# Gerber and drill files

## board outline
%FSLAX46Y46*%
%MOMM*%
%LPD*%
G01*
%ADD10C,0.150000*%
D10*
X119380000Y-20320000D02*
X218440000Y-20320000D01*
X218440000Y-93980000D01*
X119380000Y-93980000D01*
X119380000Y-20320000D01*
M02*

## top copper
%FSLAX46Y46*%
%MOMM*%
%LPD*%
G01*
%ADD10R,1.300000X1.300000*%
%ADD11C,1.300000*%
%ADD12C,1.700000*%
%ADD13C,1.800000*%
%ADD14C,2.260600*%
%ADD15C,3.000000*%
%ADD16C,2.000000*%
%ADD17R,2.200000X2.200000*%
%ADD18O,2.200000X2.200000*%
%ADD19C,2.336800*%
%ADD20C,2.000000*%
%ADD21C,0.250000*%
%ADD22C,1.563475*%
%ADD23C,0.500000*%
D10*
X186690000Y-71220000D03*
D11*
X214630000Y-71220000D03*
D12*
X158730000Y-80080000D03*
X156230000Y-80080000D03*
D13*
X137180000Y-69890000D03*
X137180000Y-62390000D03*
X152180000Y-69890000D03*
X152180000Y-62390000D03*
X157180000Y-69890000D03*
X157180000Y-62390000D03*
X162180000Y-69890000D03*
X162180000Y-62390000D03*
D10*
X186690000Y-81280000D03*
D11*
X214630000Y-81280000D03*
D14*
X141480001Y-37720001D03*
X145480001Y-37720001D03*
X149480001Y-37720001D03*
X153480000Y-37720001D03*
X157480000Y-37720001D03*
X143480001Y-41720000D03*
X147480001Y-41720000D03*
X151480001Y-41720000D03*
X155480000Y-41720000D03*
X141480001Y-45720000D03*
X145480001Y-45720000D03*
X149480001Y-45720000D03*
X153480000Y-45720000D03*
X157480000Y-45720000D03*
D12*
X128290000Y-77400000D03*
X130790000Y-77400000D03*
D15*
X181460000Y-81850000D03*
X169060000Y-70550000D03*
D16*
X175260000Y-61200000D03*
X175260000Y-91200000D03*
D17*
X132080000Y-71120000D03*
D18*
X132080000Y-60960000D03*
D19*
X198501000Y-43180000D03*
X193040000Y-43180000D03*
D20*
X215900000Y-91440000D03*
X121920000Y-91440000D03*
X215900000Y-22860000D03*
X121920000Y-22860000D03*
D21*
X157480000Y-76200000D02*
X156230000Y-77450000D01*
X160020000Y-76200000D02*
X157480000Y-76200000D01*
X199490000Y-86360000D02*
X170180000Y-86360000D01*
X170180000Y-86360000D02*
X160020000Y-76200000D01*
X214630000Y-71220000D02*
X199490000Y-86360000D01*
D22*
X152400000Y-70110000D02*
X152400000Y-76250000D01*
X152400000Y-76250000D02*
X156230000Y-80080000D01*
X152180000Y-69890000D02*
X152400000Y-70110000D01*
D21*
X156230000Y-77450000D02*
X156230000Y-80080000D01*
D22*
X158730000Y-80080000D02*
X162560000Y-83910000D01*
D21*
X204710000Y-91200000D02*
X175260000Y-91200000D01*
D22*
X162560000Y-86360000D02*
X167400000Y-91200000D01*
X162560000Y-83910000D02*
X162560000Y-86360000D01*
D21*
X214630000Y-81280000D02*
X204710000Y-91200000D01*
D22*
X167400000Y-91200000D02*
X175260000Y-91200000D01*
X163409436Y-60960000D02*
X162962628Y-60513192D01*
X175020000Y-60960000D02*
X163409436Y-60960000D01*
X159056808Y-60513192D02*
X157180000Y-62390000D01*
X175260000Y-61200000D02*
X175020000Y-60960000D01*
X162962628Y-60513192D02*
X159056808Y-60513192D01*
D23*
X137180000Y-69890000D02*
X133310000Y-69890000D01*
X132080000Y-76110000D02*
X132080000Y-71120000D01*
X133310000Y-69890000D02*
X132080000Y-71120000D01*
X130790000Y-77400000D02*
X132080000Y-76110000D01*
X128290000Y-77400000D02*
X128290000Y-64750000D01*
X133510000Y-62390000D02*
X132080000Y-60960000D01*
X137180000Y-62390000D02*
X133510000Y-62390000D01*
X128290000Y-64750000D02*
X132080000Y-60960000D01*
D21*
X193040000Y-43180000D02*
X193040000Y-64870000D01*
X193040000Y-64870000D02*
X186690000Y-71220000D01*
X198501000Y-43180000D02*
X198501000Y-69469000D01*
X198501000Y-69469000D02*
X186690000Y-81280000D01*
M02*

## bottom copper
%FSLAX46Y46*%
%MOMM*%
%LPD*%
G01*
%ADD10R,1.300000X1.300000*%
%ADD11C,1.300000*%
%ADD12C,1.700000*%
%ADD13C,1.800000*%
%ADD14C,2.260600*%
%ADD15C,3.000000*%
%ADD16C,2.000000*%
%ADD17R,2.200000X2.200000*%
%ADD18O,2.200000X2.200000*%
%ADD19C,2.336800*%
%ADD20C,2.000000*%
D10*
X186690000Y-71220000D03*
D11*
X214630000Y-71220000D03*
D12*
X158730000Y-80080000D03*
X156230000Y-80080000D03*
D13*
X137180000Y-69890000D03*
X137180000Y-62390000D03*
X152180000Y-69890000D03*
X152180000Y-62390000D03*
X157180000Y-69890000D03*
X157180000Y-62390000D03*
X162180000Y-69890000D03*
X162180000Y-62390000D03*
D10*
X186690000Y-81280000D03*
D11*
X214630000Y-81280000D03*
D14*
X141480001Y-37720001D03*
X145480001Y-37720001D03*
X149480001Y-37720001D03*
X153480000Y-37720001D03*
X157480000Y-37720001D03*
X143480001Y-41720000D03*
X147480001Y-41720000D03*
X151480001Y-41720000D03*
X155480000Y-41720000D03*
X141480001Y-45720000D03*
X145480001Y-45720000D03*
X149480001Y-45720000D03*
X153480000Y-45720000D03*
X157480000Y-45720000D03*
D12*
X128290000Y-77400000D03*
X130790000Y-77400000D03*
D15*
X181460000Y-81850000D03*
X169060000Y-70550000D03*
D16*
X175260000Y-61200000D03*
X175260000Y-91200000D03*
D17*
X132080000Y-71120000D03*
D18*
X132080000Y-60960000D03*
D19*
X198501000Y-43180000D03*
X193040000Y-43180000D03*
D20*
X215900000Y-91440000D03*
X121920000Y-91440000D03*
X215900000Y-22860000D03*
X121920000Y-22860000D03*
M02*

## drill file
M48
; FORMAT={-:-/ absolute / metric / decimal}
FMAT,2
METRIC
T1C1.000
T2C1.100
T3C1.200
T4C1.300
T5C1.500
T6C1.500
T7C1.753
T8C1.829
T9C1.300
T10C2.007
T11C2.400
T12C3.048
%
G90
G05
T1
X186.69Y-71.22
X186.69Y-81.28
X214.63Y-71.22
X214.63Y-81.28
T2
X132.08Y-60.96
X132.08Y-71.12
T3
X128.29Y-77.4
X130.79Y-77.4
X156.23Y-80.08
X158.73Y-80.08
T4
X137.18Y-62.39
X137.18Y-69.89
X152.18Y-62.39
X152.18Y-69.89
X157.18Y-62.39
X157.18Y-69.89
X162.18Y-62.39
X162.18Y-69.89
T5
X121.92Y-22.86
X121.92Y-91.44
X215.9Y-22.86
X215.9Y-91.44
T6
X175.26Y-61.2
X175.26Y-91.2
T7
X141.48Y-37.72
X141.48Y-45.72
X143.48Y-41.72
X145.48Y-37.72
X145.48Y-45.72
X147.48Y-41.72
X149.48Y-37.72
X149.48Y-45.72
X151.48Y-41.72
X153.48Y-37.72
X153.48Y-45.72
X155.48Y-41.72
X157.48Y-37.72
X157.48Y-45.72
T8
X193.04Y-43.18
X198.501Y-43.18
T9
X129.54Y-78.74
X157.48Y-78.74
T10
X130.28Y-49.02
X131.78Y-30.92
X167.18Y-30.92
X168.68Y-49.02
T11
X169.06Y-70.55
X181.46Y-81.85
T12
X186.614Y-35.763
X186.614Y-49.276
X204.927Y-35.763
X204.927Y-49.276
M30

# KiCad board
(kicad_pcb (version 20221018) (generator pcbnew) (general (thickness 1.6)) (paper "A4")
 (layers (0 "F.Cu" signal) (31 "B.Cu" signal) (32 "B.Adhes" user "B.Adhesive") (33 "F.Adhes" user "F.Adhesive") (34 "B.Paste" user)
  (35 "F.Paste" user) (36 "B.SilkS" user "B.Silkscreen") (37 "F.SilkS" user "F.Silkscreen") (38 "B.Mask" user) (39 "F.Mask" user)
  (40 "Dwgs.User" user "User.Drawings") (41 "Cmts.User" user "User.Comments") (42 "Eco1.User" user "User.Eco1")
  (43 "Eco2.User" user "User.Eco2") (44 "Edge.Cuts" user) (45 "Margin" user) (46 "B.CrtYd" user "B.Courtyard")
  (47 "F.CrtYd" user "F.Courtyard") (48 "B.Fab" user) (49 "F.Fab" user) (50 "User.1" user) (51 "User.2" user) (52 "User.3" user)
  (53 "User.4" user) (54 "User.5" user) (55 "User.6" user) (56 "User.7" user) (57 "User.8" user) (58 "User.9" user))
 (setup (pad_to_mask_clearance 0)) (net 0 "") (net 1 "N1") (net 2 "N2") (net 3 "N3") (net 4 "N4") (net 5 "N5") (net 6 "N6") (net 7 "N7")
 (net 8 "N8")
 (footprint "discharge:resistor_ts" (layer "F.Cu") (at 190.627 67.4735)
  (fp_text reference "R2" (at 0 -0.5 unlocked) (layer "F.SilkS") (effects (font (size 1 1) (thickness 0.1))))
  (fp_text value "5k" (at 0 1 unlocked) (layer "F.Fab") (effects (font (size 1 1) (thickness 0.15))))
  (pad "1" thru_hole rect (at -3.937 3.7465) (size 1.3 1.3) (drill 1) (layers "*.Cu" "*.Mask") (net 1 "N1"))
  (pad "2" thru_hole circle (at 24.003 3.7465) (size 1.3 1.3) (drill 1) (layers "*.Cu" "*.Mask") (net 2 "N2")))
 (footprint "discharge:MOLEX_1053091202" (layer "F.Cu") (at 158.73 80.08 180)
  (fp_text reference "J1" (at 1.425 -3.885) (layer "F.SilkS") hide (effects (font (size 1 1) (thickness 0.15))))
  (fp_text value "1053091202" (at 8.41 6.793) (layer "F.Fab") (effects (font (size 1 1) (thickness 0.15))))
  (pad "" np_thru_hole circle (at 1.25 1.34 180) (size 1.3 1.3) (drill 1.3) (layers "*.Cu" "*.Mask"))
  (pad "1" thru_hole circle (at 0 0 180) (size 1.7 1.7) (drill 1.2) (layers "*.Cu") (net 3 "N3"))
  (pad "2" thru_hole circle (at 2.5 0 180) (size 1.7 1.7) (drill 1.2) (layers "*.Cu") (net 2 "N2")))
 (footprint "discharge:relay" (layer "F.Cu") (at 134.68 72.39 90)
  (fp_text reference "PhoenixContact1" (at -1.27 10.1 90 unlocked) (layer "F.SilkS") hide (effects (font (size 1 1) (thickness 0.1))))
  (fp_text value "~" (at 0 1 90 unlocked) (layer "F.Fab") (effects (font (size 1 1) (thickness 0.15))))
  (pad "1" thru_hole circle (at 2.5 2.5 90) (size 1.8 1.8) (drill 1.3) (layers "*.Cu" "*.Mask") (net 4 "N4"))
  (pad "2" thru_hole circle (at 10 2.5 90) (size 1.8 1.8) (drill 1.3) (layers "*.Cu" "*.Mask") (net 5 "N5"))
  (pad "3" thru_hole circle (at 2.5 17.5 90) (size 1.8 1.8) (drill 1.3) (layers "*.Cu" "*.Mask") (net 2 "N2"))
  (pad "3" thru_hole circle (at 10 17.5 90) (size 1.8 1.8) (drill 1.3) (layers "*.Cu" "*.Mask") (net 2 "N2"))
  (pad "4" thru_hole circle (at 2.5 22.5 90) (size 1.8 1.8) (drill 1.3) (layers "*.Cu" "*.Mask") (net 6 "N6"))
  (pad "4" thru_hole circle (at 10 22.5 90) (size 1.8 1.8) (drill 1.3) (layers "*.Cu" "*.Mask") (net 6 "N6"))
  (pad "5" thru_hole circle (at 2.5 27.5 90) (size 1.8 1.8) (drill 1.3) (layers "*.Cu" "*.Mask") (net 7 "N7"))
  (pad "5" thru_hole circle (at 10 27.5 90) (size 1.8 1.8) (drill 1.3) (layers "*.Cu" "*.Mask") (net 7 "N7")))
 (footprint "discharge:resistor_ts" (layer "F.Cu") (at 190.627 77.5335)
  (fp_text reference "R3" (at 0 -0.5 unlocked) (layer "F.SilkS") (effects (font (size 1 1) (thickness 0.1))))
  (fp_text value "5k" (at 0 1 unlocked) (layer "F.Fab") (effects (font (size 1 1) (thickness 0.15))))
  (pad "1" thru_hole rect (at -3.937 3.7465) (size 1.3 1.3) (drill 1) (layers "*.Cu" "*.Mask") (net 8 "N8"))
  (pad "2" thru_hole circle (at 24.003 3.7465) (size 1.3 1.3) (drill 1) (layers "*.Cu" "*.Mask") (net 3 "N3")))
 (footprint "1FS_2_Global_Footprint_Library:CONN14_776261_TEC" (layer "F.Cu") (at 157.48 45.72)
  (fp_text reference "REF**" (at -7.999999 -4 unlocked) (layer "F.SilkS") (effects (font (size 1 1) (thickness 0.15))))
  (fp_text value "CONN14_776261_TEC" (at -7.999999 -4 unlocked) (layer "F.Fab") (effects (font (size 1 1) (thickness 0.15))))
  (pad "" np_thru_hole circle (at -27.199999 3.300001) (size 2.0066 2.0066) (drill 2.0066) (layers "*.Cu" "*.Mask"))
  (pad "" np_thru_hole circle (at -25.700003 -14.799999) (size 2.0066 2.0066) (drill 2.0066) (layers "*.Cu" "*.Mask"))
  (pad "" np_thru_hole circle (at 9.700004 -14.799999) (size 2.0066 2.0066) (drill 2.0066) (layers "*.Cu" "*.Mask"))
  (pad "" np_thru_hole circle (at 11.200001 3.300001) (size 2.0066 2.0066) (drill 2.0066) (layers "*.Cu" "*.Mask"))
  (pad "1" thru_hole circle (at -15.999999 -7.999999) (size 2.2606 2.2606) (drill 1.7526) (layers "*.Cu" "*.Mask"))
  (pad "2" thru_hole circle (at -11.999999 -7.999999) (size 2.2606 2.2606) (drill 1.7526) (layers "*.Cu" "*.Mask"))
  (pad "3" thru_hole circle (at -7.999999 -7.999999) (size 2.2606 2.2606) (drill 1.7526) (layers "*.Cu" "*.Mask"))
  (pad "4" thru_hole circle (at -4 -7.999999) (size 2.2606 2.2606) (drill 1.7526) (layers "*.Cu" "*.Mask"))
  (pad "5" thru_hole circle (at 0 -7.999999) (size 2.2606 2.2606) (drill 1.7526) (layers "*.Cu" "*.Mask"))
  (pad "6" thru_hole circle (at -13.999999 -4) (size 2.2606 2.2606) (drill 1.7526) (layers "*.Cu" "*.Mask"))
  (pad "7" thru_hole circle (at -9.999999 -4) (size 2.2606 2.2606) (drill 1.7526) (layers "*.Cu" "*.Mask"))
  (pad "8" thru_hole circle (at -5.999999 -4) (size 2.2606 2.2606) (drill 1.7526) (layers "*.Cu" "*.Mask"))
  (pad "9" thru_hole circle (at -2 -4) (size 2.2606 2.2606) (drill 1.7526) (layers "*.Cu" "*.Mask"))
  (pad "10" thru_hole circle (at -15.999999 0) (size 2.2606 2.2606) (drill 1.7526) (layers "*.Cu" "*.Mask"))
  (pad "11" thru_hole circle (at -11.999999 0) (size 2.2606 2.2606) (drill 1.7526) (layers "*.Cu" "*.Mask"))
  (pad "12" thru_hole circle (at -7.999999 0) (size 2.2606 2.2606) (drill 1.7526) (layers "*.Cu" "*.Mask"))
  (pad "13" thru_hole circle (at -4 0) (size 2.2606 2.2606) (drill 1.7526) (layers "*.Cu" "*.Mask"))
  (pad "14" thru_hole circle (at 0 0) (size 2.2606 2.2606) (drill 1.7526) (layers "*.Cu" "*.Mask")))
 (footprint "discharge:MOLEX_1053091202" (layer "F.Cu") (at 128.29 77.4)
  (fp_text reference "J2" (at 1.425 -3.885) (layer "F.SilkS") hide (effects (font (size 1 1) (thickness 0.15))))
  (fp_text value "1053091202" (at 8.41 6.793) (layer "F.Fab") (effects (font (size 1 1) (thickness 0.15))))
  (pad "" np_thru_hole circle (at 1.25 1.34) (size 1.3 1.3) (drill 1.3) (layers "*.Cu" "*.Mask"))
  (pad "1" thru_hole circle (at 0 0) (size 1.7 1.7) (drill 1.2) (layers "*.Cu") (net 5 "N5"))
  (pad "2" thru_hole circle (at 2.5 0) (size 1.7 1.7) (drill 1.2) (layers "*.Cu") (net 4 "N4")))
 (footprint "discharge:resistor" (layer "F.Cu") (at 166.76 84.7 90)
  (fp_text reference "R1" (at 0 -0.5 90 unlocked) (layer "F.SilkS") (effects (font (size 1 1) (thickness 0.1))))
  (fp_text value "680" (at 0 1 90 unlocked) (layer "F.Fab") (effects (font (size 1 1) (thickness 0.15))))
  (pad "" np_thru_hole circle (at 2.85 14.7 90) (size 3 3) (drill 2.4) (layers "F&B.Cu" "*.Mask"))
  (pad "" np_thru_hole circle (at 14.15 2.3 90) (size 3 3) (drill 2.4) (layers "F&B.Cu" "*.Mask"))
  (pad "1" thru_hole circle (at 23.5 8.5 90) (size 2 2) (drill 1.5) (layers "*.Cu" "*.Mask") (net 6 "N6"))
  (pad "2" thru_hole circle (at -6.5 8.5 90) (size 2 2) (drill 1.5) (layers "*.Cu" "*.Mask") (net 3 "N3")))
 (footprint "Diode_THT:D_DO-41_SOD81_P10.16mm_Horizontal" (layer "F.Cu") (at 132.08 71.12 90)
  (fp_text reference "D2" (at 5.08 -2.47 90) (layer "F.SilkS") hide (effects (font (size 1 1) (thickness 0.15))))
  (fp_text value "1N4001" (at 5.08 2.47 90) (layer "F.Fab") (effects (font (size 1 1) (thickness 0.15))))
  (pad "1" thru_hole rect (at 0 0 90) (size 2.2 2.2) (drill 1.1) (layers "*.Cu" "*.Mask") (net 4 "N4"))
  (pad "2" thru_hole oval (at 10.16 0 90) (size 2.2 2.2) (drill 1.1) (layers "*.Cu" "*.Mask") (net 5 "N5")))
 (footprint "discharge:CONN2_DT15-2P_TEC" (layer "F.Cu") (at 193.04 43.18)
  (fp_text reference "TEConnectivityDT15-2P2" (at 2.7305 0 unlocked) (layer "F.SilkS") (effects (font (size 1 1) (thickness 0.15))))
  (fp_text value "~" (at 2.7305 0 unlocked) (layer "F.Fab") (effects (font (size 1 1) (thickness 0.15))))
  (pad "" np_thru_hole circle (at -6.4262 -7.4168) (size 3.048 3.048) (drill 3.048) (layers))
  (pad "" np_thru_hole circle (at -6.4262 6.096) (size 3.048 3.048) (drill 3.048) (layers))
  (pad "" np_thru_hole circle (at 11.8872 -7.4168) (size 3.048 3.048) (drill 3.048) (layers))
  (pad "" np_thru_hole circle (at 11.8872 6.096) (size 3.048 3.048) (drill 3.048) (layers))
  (pad "1" thru_hole circle (at 5.461 0) (size 2.3368 2.3368) (drill 1.8288) (layers "*.Cu" "*.Mask") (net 8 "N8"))
  (pad "2" thru_hole circle (at 0 0) (size 2.3368 2.3368) (drill 1.8288) (layers "*.Cu" "*.Mask") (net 1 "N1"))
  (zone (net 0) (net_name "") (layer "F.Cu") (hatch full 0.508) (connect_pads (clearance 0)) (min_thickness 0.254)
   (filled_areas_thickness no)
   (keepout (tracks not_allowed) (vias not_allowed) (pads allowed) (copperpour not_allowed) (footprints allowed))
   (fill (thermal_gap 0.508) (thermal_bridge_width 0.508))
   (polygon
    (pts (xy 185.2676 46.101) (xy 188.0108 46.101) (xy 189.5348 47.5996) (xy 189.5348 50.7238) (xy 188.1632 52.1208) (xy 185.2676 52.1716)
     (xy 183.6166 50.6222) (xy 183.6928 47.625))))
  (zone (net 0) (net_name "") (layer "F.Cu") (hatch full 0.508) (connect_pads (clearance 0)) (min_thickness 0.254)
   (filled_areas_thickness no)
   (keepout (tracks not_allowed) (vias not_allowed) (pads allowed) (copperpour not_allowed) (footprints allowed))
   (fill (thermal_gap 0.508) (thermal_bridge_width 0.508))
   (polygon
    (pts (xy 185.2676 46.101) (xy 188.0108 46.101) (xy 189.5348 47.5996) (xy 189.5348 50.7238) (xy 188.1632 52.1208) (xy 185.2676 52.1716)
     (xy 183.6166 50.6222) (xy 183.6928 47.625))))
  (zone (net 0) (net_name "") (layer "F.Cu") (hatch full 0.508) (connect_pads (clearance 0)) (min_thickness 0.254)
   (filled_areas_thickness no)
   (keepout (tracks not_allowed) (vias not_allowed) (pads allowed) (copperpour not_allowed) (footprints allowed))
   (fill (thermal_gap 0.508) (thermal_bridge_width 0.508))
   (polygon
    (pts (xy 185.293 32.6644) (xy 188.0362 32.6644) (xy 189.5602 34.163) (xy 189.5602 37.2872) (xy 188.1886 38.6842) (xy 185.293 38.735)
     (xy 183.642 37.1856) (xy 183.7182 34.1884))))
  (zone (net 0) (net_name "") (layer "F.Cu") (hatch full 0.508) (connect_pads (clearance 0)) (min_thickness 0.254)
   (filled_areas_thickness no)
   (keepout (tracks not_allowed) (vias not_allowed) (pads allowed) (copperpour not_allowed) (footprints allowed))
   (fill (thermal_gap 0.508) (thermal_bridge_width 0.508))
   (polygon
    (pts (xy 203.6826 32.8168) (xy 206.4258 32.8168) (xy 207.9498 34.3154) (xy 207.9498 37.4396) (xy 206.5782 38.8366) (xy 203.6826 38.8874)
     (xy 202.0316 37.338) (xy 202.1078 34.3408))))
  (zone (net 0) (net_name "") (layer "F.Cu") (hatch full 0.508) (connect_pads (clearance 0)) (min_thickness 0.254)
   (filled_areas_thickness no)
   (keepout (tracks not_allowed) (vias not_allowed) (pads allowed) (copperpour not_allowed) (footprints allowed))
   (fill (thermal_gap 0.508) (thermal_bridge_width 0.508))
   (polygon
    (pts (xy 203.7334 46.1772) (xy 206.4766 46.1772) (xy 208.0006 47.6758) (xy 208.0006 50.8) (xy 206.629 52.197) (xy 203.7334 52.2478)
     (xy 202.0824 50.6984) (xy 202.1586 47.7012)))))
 (gr_rect (start 119.38 20.32) (end 218.44 93.98) (stroke (width 0.15) (type default)) (fill none) (layer "Edge.Cuts"))
 (via (at 215.9 91.44) (size 2) (drill 1.5) (layers "F.Cu" "B.Cu") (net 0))
 (via (at 121.92 91.44) (size 2) (drill 1.5) (layers "F.Cu" "B.Cu") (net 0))
 (via (at 215.9 22.86) (size 2) (drill 1.5) (layers "F.Cu" "B.Cu") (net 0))
 (via (at 121.92 22.86) (size 2) (drill 1.5) (layers "F.Cu" "B.Cu") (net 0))
 (segment (start 157.48 76.2) (end 156.23 77.45) (width 0.25) (layer "F.Cu") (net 2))
 (segment (start 160.02 76.2) (end 157.48 76.2) (width 0.25) (layer "F.Cu") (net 2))
 (segment (start 199.49 86.36) (end 170.18 86.36) (width 0.25) (layer "F.Cu") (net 2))
 (segment (start 170.18 86.36) (end 160.02 76.2) (width 0.25) (layer "F.Cu") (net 2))
 (segment (start 214.63 71.22) (end 199.49 86.36) (width 0.25) (layer "F.Cu") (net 2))
 (segment (start 152.4 70.11) (end 152.4 76.25) (width 1.563475) (layer "F.Cu") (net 2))
 (segment (start 152.4 76.25) (end 156.23 80.08) (width 1.563475) (layer "F.Cu") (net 2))
 (segment (start 152.18 69.89) (end 152.4 70.11) (width 1.563475) (layer "F.Cu") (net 2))
 (segment (start 156.23 77.45) (end 156.23 80.08) (width 0.25) (layer "F.Cu") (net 2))
 (segment (start 158.73 80.08) (end 162.56 83.91) (width 1.563475) (layer "F.Cu") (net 3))
 (segment (start 204.71 91.2) (end 175.26 91.2) (width 0.25) (layer "F.Cu") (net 3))
 (segment (start 162.56 86.36) (end 167.4 91.2) (width 1.563475) (layer "F.Cu") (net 3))
 (segment (start 162.56 83.91) (end 162.56 86.36) (width 1.563475) (layer "F.Cu") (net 3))
 (segment (start 214.63 81.28) (end 204.71 91.2) (width 0.25) (layer "F.Cu") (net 3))
 (segment (start 167.4 91.2) (end 175.26 91.2) (width 1.563475) (layer "F.Cu") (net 3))
 (segment (start 163.409436 60.96) (end 162.962628 60.513192) (width 1.563475) (layer "F.Cu") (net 6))
 (segment (start 175.02 60.96) (end 163.409436 60.96) (width 1.563475) (layer "F.Cu") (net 6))
 (segment (start 159.056808 60.513192) (end 157.18 62.39) (width 1.563475) (layer "F.Cu") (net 6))
 (segment (start 175.26 61.2) (end 175.02 60.96) (width 1.563475) (layer "F.Cu") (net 6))
 (segment (start 162.962628 60.513192) (end 159.056808 60.513192) (width 1.563475) (layer "F.Cu") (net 6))
 (segment (start 137.18 69.89) (end 133.31 69.89) (width 0.5) (layer "F.Cu") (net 4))
 (segment (start 132.08 76.11) (end 132.08 71.12) (width 0.5) (layer "F.Cu") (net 4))
 (segment (start 133.31 69.89) (end 132.08 71.12) (width 0.5) (layer "F.Cu") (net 4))
 (segment (start 130.79 77.4) (end 132.08 76.11) (width 0.5) (layer "F.Cu") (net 4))
 (segment (start 128.29 77.4) (end 128.29 64.75) (width 0.5) (layer "F.Cu") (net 5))
 (segment (start 133.51 62.39) (end 132.08 60.96) (width 0.5) (layer "F.Cu") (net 5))
 (segment (start 137.18 62.39) (end 133.51 62.39) (width 0.5) (layer "F.Cu") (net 5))
 (segment (start 128.29 64.75) (end 132.08 60.96) (width 0.5) (layer "F.Cu") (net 5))
 (segment (start 193.04 43.18) (end 193.04 64.87) (width 0.25) (layer "F.Cu") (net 1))
 (segment (start 193.04 64.87) (end 186.69 71.22) (width 0.25) (layer "F.Cu") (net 1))
 (segment (start 198.501 43.18) (end 198.501 69.469) (width 0.25) (layer "F.Cu") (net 8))
 (segment (start 198.501 69.469) (end 186.69 81.28) (width 0.25) (layer "F.Cu") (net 8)))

